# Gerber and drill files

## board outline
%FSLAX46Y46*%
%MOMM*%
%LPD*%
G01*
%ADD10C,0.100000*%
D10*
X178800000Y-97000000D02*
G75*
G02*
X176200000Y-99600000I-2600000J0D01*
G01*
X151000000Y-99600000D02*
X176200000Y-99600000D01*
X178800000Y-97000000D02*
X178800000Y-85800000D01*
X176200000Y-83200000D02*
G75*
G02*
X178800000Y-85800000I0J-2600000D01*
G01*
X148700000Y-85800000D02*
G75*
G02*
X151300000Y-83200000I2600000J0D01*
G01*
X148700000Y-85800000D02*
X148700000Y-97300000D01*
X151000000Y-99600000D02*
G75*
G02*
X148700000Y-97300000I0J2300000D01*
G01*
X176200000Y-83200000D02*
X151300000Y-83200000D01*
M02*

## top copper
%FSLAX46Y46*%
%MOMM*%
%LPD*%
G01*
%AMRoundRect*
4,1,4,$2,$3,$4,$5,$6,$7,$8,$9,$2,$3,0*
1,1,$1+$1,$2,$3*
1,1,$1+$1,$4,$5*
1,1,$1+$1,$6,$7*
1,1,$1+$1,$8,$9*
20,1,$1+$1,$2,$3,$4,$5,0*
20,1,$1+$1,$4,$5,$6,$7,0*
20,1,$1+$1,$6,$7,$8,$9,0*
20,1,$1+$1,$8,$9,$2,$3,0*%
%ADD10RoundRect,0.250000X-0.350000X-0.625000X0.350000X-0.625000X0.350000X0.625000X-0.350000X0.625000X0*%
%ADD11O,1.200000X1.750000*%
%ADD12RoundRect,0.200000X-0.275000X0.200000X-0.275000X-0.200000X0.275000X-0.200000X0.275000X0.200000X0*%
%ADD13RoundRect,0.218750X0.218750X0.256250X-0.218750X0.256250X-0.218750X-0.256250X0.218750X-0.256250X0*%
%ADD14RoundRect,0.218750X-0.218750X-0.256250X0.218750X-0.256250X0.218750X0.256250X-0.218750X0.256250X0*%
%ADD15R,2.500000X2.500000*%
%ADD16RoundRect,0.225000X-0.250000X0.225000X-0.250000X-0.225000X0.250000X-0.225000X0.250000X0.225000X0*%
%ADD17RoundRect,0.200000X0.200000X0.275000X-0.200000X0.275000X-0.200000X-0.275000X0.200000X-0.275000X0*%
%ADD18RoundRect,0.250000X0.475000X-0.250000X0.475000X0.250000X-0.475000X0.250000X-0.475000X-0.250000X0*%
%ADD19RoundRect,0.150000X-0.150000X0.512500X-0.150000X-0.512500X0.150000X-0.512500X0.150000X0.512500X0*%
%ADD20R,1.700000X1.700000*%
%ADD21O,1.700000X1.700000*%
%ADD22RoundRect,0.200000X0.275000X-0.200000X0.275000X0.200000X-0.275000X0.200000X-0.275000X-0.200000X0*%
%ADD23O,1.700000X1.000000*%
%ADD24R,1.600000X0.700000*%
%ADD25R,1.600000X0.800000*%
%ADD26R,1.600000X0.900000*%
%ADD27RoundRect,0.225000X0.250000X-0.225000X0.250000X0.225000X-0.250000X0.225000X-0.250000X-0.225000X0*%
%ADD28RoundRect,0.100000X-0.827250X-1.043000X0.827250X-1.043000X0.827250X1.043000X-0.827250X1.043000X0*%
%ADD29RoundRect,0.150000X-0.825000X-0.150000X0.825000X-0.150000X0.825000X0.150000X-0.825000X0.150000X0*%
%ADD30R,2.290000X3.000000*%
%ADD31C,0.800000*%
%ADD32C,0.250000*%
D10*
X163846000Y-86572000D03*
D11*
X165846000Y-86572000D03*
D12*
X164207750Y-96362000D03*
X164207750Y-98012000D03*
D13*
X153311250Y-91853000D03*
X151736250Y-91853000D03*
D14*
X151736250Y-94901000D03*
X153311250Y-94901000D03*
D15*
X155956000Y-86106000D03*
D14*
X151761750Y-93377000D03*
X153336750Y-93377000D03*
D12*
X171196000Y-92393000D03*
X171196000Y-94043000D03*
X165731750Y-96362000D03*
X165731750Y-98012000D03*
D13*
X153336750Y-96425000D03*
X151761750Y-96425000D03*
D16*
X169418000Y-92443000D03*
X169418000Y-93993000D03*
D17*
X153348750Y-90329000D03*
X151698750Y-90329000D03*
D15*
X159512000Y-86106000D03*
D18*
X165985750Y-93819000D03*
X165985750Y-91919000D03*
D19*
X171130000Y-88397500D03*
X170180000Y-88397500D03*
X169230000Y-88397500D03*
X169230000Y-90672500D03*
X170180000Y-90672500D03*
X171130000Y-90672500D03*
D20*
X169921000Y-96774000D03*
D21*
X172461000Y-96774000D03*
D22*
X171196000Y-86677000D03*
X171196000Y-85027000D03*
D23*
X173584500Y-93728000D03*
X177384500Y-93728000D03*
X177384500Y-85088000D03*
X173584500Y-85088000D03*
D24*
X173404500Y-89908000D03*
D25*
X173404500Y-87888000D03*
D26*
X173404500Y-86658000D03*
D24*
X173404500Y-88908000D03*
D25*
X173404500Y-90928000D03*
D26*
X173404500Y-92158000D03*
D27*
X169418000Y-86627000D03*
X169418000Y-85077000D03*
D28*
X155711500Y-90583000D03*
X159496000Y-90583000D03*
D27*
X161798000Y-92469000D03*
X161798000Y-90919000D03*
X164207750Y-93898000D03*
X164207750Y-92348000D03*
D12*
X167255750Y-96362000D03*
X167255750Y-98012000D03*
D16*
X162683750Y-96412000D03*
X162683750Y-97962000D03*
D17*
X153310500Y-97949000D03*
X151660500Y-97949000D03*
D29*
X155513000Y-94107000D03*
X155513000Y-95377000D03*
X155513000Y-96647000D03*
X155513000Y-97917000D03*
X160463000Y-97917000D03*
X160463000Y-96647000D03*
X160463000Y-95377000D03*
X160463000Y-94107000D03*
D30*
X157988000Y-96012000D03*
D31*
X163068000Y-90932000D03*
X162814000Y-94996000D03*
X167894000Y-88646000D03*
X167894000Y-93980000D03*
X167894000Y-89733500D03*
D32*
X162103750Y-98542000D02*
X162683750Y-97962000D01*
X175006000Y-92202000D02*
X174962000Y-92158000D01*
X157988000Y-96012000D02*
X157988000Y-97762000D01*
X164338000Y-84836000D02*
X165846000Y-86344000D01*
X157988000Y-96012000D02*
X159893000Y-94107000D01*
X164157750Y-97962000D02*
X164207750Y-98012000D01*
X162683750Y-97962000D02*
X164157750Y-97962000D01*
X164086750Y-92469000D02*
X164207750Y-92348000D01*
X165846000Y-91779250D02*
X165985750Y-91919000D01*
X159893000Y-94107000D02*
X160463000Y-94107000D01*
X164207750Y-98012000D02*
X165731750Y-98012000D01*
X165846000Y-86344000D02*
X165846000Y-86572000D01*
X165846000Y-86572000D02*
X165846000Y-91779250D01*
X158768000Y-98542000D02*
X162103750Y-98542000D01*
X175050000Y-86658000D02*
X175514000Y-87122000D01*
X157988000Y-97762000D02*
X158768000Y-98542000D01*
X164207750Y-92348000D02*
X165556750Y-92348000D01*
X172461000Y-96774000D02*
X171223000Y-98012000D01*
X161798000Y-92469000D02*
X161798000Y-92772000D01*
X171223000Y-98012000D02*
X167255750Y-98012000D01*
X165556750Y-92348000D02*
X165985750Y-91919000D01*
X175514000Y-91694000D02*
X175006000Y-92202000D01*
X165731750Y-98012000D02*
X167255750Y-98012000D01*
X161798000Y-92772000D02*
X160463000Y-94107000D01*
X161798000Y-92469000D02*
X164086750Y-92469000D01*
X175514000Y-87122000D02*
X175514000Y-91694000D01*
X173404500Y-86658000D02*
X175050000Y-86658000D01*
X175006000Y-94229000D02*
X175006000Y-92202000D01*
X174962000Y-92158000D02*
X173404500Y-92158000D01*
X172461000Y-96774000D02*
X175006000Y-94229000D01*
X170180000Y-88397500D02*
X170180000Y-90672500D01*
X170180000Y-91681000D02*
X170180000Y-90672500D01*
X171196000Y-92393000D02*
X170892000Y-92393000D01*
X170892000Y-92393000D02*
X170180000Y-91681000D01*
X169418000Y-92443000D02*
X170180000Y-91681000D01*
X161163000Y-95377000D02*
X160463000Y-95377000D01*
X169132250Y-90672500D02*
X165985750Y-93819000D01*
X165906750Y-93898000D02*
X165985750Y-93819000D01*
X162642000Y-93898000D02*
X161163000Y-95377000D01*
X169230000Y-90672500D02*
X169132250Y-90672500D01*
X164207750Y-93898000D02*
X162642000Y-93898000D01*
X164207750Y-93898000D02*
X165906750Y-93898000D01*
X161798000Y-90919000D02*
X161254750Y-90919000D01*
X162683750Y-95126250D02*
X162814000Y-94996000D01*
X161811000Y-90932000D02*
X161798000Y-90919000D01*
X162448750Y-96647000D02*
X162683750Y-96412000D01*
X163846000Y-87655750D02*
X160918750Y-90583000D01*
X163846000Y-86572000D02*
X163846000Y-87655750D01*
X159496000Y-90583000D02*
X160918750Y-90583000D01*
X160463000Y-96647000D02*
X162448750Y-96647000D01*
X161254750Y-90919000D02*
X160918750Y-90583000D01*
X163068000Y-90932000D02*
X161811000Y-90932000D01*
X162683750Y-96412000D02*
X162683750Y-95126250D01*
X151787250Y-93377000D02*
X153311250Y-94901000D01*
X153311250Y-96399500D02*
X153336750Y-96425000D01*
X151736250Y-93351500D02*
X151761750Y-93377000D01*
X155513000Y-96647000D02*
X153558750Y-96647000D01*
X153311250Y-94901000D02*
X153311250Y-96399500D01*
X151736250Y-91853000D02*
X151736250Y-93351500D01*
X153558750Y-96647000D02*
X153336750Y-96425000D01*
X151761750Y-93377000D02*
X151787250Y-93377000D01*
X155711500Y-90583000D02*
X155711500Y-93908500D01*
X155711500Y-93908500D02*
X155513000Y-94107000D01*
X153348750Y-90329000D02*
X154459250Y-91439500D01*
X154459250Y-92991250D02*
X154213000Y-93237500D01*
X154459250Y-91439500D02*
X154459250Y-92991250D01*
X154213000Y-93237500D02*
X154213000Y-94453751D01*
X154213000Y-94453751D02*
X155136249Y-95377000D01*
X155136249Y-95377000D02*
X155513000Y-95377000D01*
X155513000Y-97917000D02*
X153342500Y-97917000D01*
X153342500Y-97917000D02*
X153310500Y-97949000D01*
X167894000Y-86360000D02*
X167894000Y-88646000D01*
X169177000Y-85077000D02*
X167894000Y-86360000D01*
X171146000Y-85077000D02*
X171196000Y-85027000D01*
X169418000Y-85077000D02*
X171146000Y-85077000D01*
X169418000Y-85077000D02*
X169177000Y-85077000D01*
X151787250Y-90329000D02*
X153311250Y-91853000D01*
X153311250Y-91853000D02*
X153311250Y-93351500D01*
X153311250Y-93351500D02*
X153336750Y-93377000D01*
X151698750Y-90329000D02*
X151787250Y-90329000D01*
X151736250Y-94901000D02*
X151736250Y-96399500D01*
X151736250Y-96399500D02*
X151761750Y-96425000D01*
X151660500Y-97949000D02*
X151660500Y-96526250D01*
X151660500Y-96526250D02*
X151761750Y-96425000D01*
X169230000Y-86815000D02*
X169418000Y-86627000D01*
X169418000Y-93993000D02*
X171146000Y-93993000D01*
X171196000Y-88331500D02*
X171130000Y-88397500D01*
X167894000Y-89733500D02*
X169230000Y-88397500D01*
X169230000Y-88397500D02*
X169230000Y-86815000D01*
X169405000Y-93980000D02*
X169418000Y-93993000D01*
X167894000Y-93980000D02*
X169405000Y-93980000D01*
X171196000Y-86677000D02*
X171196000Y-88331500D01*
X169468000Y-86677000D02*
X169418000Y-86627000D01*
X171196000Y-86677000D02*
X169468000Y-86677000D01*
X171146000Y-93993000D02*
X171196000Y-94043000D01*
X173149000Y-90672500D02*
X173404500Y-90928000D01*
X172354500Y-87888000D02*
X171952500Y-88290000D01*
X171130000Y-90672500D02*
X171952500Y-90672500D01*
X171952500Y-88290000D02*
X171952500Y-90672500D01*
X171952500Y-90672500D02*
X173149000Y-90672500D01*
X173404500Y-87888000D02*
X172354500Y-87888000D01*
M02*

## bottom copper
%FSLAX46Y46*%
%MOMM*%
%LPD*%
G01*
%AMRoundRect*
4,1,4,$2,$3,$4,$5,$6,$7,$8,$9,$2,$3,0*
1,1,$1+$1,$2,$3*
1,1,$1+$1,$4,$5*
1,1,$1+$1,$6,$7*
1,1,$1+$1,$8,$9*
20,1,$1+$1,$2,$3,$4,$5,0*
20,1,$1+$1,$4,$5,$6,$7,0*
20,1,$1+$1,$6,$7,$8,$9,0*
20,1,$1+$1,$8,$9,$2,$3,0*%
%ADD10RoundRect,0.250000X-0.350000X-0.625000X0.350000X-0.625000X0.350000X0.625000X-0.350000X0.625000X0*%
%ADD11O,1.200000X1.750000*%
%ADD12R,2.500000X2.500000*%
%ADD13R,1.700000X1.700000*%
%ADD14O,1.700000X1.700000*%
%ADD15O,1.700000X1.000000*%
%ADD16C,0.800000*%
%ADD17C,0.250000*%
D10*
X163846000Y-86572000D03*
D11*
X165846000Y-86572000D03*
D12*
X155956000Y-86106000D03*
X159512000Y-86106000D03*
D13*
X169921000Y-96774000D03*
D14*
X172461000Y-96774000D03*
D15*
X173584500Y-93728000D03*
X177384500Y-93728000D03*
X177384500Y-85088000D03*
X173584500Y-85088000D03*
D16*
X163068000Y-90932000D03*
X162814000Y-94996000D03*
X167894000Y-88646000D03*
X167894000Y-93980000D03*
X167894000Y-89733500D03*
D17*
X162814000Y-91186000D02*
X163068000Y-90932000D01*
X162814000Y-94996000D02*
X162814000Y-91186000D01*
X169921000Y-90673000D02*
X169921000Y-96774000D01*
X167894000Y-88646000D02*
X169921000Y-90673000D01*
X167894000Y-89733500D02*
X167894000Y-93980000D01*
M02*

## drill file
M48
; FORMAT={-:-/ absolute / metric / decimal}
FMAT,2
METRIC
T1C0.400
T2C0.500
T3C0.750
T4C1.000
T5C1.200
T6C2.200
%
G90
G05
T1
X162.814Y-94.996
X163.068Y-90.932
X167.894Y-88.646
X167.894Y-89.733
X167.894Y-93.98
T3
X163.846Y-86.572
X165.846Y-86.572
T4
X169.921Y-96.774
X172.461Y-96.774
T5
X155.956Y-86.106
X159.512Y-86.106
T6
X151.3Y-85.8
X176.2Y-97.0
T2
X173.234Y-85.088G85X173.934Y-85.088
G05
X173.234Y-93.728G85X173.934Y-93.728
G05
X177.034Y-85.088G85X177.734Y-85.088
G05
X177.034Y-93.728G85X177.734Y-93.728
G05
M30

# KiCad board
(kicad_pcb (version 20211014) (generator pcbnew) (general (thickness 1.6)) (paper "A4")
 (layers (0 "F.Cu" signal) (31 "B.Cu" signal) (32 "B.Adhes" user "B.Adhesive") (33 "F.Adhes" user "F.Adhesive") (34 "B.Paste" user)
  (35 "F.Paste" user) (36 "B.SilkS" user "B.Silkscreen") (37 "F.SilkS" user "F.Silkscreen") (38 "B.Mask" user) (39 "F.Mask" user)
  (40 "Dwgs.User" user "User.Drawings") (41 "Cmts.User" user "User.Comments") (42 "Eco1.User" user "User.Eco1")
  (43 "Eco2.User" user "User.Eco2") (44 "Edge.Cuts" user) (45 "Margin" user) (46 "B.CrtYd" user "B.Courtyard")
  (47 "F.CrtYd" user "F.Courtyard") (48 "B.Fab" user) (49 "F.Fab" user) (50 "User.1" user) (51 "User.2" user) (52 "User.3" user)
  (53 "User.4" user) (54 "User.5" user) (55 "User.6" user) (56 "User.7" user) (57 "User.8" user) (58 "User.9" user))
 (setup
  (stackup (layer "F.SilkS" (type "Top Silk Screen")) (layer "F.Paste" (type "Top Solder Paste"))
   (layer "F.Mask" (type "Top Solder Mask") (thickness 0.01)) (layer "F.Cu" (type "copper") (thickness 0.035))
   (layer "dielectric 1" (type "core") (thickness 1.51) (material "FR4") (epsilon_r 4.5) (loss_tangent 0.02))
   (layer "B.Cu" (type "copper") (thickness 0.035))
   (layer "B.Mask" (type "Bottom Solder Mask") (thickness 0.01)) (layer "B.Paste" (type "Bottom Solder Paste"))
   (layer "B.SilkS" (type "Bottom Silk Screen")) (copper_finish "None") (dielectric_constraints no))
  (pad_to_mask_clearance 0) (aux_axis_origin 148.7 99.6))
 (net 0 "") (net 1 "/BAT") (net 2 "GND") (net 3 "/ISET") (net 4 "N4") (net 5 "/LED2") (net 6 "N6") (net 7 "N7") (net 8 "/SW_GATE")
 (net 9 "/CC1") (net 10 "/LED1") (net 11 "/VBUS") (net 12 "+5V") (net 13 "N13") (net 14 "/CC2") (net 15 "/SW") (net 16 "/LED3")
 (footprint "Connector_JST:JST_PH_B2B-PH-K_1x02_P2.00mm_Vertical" (layer "F.Cu") (at 163.846 86.572)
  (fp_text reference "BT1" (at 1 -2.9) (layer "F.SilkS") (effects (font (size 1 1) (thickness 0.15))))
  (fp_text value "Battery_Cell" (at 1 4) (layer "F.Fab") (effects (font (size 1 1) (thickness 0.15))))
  (pad "1" thru_hole roundrect (at 0 0) (size 1.2 1.75) (drill 0.75) (layers *.Cu *.Mask) (roundrect_rratio 0.208333) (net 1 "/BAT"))
  (pad "2" thru_hole oval (at 2 0) (size 1.2 1.75) (drill 0.75) (layers *.Cu *.Mask) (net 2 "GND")))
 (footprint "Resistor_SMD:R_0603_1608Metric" (layer "F.Cu") (at 164.20775 97.187 -90)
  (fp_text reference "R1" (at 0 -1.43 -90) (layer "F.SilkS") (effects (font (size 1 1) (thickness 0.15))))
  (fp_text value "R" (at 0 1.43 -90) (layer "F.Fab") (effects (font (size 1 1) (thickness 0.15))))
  (pad "1" smd roundrect (at -0.825 0 270) (size 0.8 0.95) (layers "F.Cu" "F.Paste" "F.Mask") (roundrect_rratio 0.25) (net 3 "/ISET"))
  (pad "2" smd roundrect (at 0.825 0 270) (size 0.8 0.95) (layers "F.Cu" "F.Paste" "F.Mask") (roundrect_rratio 0.25) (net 2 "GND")))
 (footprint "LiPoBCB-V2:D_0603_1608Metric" (layer "F.Cu") (at 152.52375 91.853 180)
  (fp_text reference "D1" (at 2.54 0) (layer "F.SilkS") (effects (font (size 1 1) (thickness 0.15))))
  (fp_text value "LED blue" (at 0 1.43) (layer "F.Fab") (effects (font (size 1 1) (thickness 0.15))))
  (pad "1" smd roundrect (at -0.7875 0 180) (size 0.875 0.95) (layers "F.Cu" "F.Paste" "F.Mask") (roundrect_rratio 0.25) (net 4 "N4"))
  (pad "2" smd roundrect (at 0.7875 0 180) (size 0.875 0.95) (layers "F.Cu" "F.Paste" "F.Mask") (roundrect_rratio 0.25) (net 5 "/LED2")))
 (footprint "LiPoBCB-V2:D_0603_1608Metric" (layer "F.Cu") (at 152.52375 94.901)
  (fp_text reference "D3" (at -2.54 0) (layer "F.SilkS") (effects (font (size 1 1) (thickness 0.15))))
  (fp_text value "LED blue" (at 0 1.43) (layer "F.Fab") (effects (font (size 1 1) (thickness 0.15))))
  (pad "1" smd roundrect (at -0.7875 0) (size 0.875 0.95) (layers "F.Cu" "F.Paste" "F.Mask") (roundrect_rratio 0.25) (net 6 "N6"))
  (pad "2" smd roundrect (at 0.7875 0) (size 0.875 0.95) (layers "F.Cu" "F.Paste" "F.Mask") (roundrect_rratio 0.25) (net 5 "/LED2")))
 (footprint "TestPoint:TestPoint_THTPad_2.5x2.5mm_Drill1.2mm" (layer "F.Cu") (at 155.956 86.106)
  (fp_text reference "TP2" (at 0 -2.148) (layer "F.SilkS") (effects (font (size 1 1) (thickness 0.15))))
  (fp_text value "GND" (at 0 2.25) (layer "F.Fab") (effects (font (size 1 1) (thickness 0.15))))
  (pad "1" thru_hole rect (at 0 0) (size 2.5 2.5) (drill 1.2) (layers *.Cu *.Mask) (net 2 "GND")))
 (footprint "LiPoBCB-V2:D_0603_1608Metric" (layer "F.Cu") (at 152.54925 93.377)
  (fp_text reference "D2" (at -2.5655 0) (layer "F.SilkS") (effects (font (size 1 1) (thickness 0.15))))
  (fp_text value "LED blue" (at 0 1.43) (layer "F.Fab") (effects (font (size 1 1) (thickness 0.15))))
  (pad "1" smd roundrect (at -0.7875 0) (size 0.875 0.95) (layers "F.Cu" "F.Paste" "F.Mask") (roundrect_rratio 0.25) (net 5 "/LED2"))
  (pad "2" smd roundrect (at 0.7875 0) (size 0.875 0.95) (layers "F.Cu" "F.Paste" "F.Mask") (roundrect_rratio 0.25) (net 4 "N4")))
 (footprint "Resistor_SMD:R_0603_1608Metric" (layer "F.Cu") (at 171.196 93.218 -90)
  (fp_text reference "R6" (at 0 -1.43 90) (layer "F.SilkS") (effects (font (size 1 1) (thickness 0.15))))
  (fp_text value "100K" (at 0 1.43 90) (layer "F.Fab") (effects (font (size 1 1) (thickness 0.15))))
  (pad "1" smd roundrect (at -0.825 0 270) (size 0.8 0.95) (layers "F.Cu" "F.Paste" "F.Mask") (roundrect_rratio 0.25) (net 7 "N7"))
  (pad "2" smd roundrect (at 0.825 0 270) (size 0.8 0.95) (layers "F.Cu" "F.Paste" "F.Mask") (roundrect_rratio 0.25) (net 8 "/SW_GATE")))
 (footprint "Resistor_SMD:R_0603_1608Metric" (layer "F.Cu") (at 165.73175 97.187 -90)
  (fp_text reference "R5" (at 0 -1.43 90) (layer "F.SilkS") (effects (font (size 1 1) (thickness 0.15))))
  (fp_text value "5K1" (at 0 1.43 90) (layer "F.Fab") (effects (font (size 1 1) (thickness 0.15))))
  (pad "1" smd roundrect (at -0.825 0 270) (size 0.8 0.95) (layers "F.Cu" "F.Paste" "F.Mask") (roundrect_rratio 0.25) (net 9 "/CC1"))
  (pad "2" smd roundrect (at 0.825 0 270) (size 0.8 0.95) (layers "F.Cu" "F.Paste" "F.Mask") (roundrect_rratio 0.25) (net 2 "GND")))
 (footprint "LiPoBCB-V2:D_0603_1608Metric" (layer "F.Cu") (at 152.54925 96.425 180)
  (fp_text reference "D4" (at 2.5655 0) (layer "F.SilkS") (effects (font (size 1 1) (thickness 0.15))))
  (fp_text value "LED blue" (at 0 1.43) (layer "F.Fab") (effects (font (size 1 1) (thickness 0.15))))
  (pad "1" smd roundrect (at -0.7875 0 180) (size 0.875 0.95) (layers "F.Cu" "F.Paste" "F.Mask") (roundrect_rratio 0.25) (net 5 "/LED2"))
  (pad "2" smd roundrect (at 0.7875 0 180) (size 0.875 0.95) (layers "F.Cu" "F.Paste" "F.Mask") (roundrect_rratio 0.25) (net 6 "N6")))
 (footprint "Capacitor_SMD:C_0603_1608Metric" (layer "F.Cu") (at 169.418 93.218 -90)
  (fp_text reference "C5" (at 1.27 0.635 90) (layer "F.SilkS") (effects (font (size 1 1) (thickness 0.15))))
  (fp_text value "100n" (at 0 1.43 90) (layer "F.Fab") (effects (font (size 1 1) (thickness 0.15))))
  (pad "1" smd roundrect (at -0.775 0 270) (size 0.9 0.95) (layers "F.Cu" "F.Paste" "F.Mask") (roundrect_rratio 0.25) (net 7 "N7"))
  (pad "2" smd roundrect (at 0.775 0 270) (size 0.9 0.95) (layers "F.Cu" "F.Paste" "F.Mask") (roundrect_rratio 0.25) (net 8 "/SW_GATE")))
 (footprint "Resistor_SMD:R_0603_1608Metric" (layer "F.Cu") (at 152.52375 90.329 180)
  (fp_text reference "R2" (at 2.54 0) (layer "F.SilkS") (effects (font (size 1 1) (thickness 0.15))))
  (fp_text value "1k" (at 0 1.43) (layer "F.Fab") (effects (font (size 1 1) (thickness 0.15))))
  (pad "1" smd roundrect (at -0.825 0 180) (size 0.8 0.95) (layers "F.Cu" "F.Paste" "F.Mask") (roundrect_rratio 0.25) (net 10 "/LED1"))
  (pad "2" smd roundrect (at 0.825 0 180) (size 0.8 0.95) (layers "F.Cu" "F.Paste" "F.Mask") (roundrect_rratio 0.25) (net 4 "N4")))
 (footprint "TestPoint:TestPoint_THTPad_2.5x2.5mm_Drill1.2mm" (layer "F.Cu") (at 159.512 86.106)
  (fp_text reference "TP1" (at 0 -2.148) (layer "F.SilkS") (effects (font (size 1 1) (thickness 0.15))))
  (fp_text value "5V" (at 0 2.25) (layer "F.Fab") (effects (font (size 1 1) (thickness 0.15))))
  (pad "1" thru_hole rect (at 0 0) (size 2.5 2.5) (drill 1.2) (layers *.Cu *.Mask) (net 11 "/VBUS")))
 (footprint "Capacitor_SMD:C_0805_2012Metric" (layer "F.Cu") (at 165.98575 92.869 90)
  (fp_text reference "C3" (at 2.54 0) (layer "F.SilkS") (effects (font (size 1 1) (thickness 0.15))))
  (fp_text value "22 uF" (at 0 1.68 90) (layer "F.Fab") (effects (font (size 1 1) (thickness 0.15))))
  (pad "1" smd roundrect (at -0.95 0 90) (size 1 1.45) (layers "F.Cu" "F.Paste" "F.Mask") (roundrect_rratio 0.25) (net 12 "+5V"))
  (pad "2" smd roundrect (at 0.95 0 90) (size 1 1.45) (layers "F.Cu" "F.Paste" "F.Mask") (roundrect_rratio 0.25) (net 2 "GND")))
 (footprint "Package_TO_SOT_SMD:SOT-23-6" (layer "F.Cu") (at 170.18 89.535 -90)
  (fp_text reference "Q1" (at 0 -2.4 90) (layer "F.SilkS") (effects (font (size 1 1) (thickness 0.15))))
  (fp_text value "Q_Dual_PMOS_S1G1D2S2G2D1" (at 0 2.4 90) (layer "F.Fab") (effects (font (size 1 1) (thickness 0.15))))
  (pad "1" smd roundrect (at -1.1375 -0.95 270) (size 1.325 0.6) (layers "F.Cu" "F.Paste" "F.Mask") (roundrect_rratio 0.25)
   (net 8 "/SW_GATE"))
  (pad "2" smd roundrect (at -1.1375 0 270) (size 1.325 0.6) (layers "F.Cu" "F.Paste" "F.Mask") (roundrect_rratio 0.25) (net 7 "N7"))
  (pad "3" smd roundrect (at -1.1375 0.95 270) (size 1.325 0.6) (layers "F.Cu" "F.Paste" "F.Mask") (roundrect_rratio 0.25)
   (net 8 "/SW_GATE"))
  (pad "4" smd roundrect (at 1.1375 0.95 270) (size 1.325 0.6) (layers "F.Cu" "F.Paste" "F.Mask") (roundrect_rratio 0.25) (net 12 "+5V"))
  (pad "5" smd roundrect (at 1.1375 0 270) (size 1.325 0.6) (layers "F.Cu" "F.Paste" "F.Mask") (roundrect_rratio 0.25) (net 7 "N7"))
  (pad "6" smd roundrect (at 1.1375 -0.95 270) (size 1.325 0.6) (layers "F.Cu" "F.Paste" "F.Mask") (roundrect_rratio 0.25) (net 11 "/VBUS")))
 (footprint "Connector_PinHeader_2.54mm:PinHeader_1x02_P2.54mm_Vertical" (layer "F.Cu") (at 169.921 96.774 90)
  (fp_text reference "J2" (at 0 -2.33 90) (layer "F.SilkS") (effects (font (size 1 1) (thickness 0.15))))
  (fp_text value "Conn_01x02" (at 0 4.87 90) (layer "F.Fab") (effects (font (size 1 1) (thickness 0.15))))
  (pad "1" thru_hole rect (at 0 0 90) (size 1.7 1.7) (drill 1) (layers *.Cu *.Mask) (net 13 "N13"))
  (pad "2" thru_hole oval (at 0 2.54 90) (size 1.7 1.7) (drill 1) (layers *.Cu *.Mask) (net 2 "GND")))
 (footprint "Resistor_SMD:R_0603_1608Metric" (layer "F.Cu") (at 171.196 85.852 90)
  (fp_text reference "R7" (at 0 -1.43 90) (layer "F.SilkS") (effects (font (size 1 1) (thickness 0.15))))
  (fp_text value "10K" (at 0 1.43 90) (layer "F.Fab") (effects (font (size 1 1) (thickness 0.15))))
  (pad "1" smd roundrect (at -0.825 0 90) (size 0.8 0.95) (layers "F.Cu" "F.Paste" "F.Mask") (roundrect_rratio 0.25) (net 8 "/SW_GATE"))
  (pad "2" smd roundrect (at 0.825 0 90) (size 0.8 0.95) (layers "F.Cu" "F.Paste" "F.Mask") (roundrect_rratio 0.25) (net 13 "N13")))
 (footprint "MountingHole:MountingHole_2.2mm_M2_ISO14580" (layer "F.Cu") (at 151.3 85.8)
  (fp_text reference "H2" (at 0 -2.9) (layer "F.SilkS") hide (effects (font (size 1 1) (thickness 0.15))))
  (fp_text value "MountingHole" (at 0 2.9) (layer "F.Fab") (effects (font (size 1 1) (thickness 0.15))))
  (pad "" np_thru_hole circle (at 0 0) (size 2.2 2.2) (drill 2.2) (layers *.Cu *.Mask)))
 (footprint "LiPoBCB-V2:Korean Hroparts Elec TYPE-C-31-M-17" (layer "F.Cu") (at 173.4045 89.408 90)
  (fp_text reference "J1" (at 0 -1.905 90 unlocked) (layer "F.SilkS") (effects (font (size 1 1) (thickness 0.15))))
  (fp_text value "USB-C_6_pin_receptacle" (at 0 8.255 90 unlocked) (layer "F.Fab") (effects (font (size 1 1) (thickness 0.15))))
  (pad "1" thru_hole oval (at -4.32 0.18 90) (size 1 1.7) (drill oval 0.5 1.2) (layers *.Cu *.Mask))
  (pad "2" thru_hole oval (at -4.32 3.98 90) (size 1 1.7) (drill oval 0.5 1.2) (layers *.Cu *.Mask))
  (pad "3" thru_hole oval (at 4.32 3.98 90) (size 1 1.7) (drill oval 0.5 1.2) (layers *.Cu *.Mask))
  (pad "4" thru_hole oval (at 4.32 0.18 90) (size 1 1.7) (drill oval 0.5 1.2) (layers *.Cu *.Mask))
  (pad "A5" smd rect (at -0.5 0 90) (size 0.7 1.6) (layers "F.Cu" "F.Paste" "F.Mask") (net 9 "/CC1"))
  (pad "A9" smd rect (at 1.52 0 90) (size 0.8 1.6) (layers "F.Cu" "F.Paste" "F.Mask") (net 11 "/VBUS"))
  (pad "A12" smd rect (at 2.75 0 90) (size 0.9 1.6) (layers "F.Cu" "F.Paste" "F.Mask") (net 2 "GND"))
  (pad "B5" smd rect (at 0.5 0 90) (size 0.7 1.6) (layers "F.Cu" "F.Paste" "F.Mask") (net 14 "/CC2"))
  (pad "B9" smd rect (at -1.52 0 90) (size 0.8 1.6) (layers "F.Cu" "F.Paste" "F.Mask") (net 11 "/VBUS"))
  (pad "B12" smd rect (at -2.75 0 90) (size 0.9 1.6) (layers "F.Cu" "F.Paste" "F.Mask") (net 2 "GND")))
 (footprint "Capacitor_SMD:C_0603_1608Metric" (layer "F.Cu") (at 169.418 85.852 90)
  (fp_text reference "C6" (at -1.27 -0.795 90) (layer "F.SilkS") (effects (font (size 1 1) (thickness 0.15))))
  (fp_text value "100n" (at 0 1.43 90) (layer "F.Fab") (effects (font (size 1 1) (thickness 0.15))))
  (pad "1" smd roundrect (at -0.775 0 90) (size 0.9 0.95) (layers "F.Cu" "F.Paste" "F.Mask") (roundrect_rratio 0.25) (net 8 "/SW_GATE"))
  (pad "2" smd roundrect (at 0.775 0 90) (size 0.9 0.95) (layers "F.Cu" "F.Paste" "F.Mask") (roundrect_rratio 0.25) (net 13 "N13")))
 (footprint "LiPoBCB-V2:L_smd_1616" (layer "F.Cu") (at 157.60375 90.583)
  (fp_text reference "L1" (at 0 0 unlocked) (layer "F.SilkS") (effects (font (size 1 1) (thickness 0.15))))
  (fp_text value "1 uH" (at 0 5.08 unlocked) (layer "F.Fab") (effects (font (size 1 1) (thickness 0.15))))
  (pad "1" smd roundrect (at -1.89225 0) (size 1.8545 2.286) (layers "F.Cu" "F.Paste" "F.Mask") (roundrect_rratio 0.05392289027)
   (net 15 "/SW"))
  (pad "2" smd roundrect (at 1.89225 0) (size 1.8545 2.286) (layers "F.Cu" "F.Paste" "F.Mask") (roundrect_rratio 0.05392289027)
   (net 1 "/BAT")))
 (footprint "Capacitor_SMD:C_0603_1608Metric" (layer "F.Cu") (at 161.798 91.694 90)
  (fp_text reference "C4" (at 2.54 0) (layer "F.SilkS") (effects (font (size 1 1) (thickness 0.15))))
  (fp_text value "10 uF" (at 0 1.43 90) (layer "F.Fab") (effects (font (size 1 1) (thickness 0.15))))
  (pad "1" smd roundrect (at -0.775 0 90) (size 0.9 0.95) (layers "F.Cu" "F.Paste" "F.Mask") (roundrect_rratio 0.25) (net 2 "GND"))
  (pad "2" smd roundrect (at 0.775 0 90) (size 0.9 0.95) (layers "F.Cu" "F.Paste" "F.Mask") (roundrect_rratio 0.25) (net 1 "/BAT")))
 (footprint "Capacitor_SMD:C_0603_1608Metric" (layer "F.Cu") (at 164.20775 93.123 90)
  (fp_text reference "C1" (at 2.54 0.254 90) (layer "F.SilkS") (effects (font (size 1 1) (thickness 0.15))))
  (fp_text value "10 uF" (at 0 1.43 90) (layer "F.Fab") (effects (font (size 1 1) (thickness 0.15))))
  (pad "1" smd roundrect (at -0.775 0 90) (size 0.9 0.95) (layers "F.Cu" "F.Paste" "F.Mask") (roundrect_rratio 0.25) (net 12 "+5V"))
  (pad "2" smd roundrect (at 0.775 0 90) (size 0.9 0.95) (layers "F.Cu" "F.Paste" "F.Mask") (roundrect_rratio 0.25) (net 2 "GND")))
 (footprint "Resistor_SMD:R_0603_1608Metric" (layer "F.Cu") (at 167.25575 97.187 -90)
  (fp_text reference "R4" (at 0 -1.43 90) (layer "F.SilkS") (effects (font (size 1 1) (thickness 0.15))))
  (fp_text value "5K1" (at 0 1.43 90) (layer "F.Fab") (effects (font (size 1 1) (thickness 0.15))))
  (pad "1" smd roundrect (at -0.825 0 270) (size 0.8 0.95) (layers "F.Cu" "F.Paste" "F.Mask") (roundrect_rratio 0.25) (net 14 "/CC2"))
  (pad "2" smd roundrect (at 0.825 0 270) (size 0.8 0.95) (layers "F.Cu" "F.Paste" "F.Mask") (roundrect_rratio 0.25) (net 2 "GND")))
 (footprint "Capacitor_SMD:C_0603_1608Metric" (layer "F.Cu") (at 162.68375 97.187 -90)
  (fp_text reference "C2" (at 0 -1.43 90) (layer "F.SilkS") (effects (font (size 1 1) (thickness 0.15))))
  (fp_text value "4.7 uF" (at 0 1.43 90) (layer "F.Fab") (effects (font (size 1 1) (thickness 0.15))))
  (pad "1" smd roundrect (at -0.775 0 270) (size 0.9 0.95) (layers "F.Cu" "F.Paste" "F.Mask") (roundrect_rratio 0.25) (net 1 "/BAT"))
  (pad "2" smd roundrect (at 0.775 0 270) (size 0.9 0.95) (layers "F.Cu" "F.Paste" "F.Mask") (roundrect_rratio 0.25) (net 2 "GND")))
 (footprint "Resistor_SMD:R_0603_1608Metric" (layer "F.Cu") (at 152.4855 97.949 180)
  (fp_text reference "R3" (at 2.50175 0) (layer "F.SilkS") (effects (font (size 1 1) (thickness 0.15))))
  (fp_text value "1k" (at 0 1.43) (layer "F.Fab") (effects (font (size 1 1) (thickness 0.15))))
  (pad "1" smd roundrect (at -0.825 0 180) (size 0.8 0.95) (layers "F.Cu" "F.Paste" "F.Mask") (roundrect_rratio 0.25) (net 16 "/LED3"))
  (pad "2" smd roundrect (at 0.825 0 180) (size 0.8 0.95) (layers "F.Cu" "F.Paste" "F.Mask") (roundrect_rratio 0.25) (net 6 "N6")))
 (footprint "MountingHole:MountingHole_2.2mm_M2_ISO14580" (layer "F.Cu") (at 176.2 97)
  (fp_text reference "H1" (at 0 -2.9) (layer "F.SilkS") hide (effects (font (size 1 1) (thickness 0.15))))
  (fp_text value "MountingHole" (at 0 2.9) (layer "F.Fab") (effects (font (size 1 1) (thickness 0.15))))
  (pad "" np_thru_hole circle (at 0 0) (size 2.2 2.2) (drill 2.2) (layers *.Cu *.Mask)))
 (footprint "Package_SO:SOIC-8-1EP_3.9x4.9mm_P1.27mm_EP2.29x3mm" (layer "F.Cu") (at 157.988 96.012)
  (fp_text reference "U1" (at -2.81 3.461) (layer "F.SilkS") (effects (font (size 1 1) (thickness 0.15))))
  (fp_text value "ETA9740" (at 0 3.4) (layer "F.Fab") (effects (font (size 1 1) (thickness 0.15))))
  (pad "" smd roundrect (at 0.57 -0.75) (size 0.92 1.21) (layers "F.Paste") (roundrect_rratio 0.25))
  (pad "" smd roundrect (at 0.57 0.75) (size 0.92 1.21) (layers "F.Paste") (roundrect_rratio 0.25))
  (pad "" smd roundrect (at -0.57 -0.75) (size 0.92 1.21) (layers "F.Paste") (roundrect_rratio 0.25))
  (pad "" smd roundrect (at -0.57 0.75) (size 0.92 1.21) (layers "F.Paste") (roundrect_rratio 0.25))
  (pad "1" smd roundrect (at -2.475 -1.905) (size 1.95 0.6) (layers "F.Cu" "F.Paste" "F.Mask") (roundrect_rratio 0.25) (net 15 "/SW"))
  (pad "2" smd roundrect (at -2.475 -0.635) (size 1.95 0.6) (layers "F.Cu" "F.Paste" "F.Mask") (roundrect_rratio 0.25) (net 10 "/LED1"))
  (pad "3" smd roundrect (at -2.475 0.635) (size 1.95 0.6) (layers "F.Cu" "F.Paste" "F.Mask") (roundrect_rratio 0.25) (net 5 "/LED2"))
  (pad "4" smd roundrect (at -2.475 1.905) (size 1.95 0.6) (layers "F.Cu" "F.Paste" "F.Mask") (roundrect_rratio 0.25) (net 16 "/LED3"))
  (pad "5" smd roundrect (at 2.475 1.905) (size 1.95 0.6) (layers "F.Cu" "F.Paste" "F.Mask") (roundrect_rratio 0.25) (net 3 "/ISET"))
  (pad "6" smd roundrect (at 2.475 0.635) (size 1.95 0.6) (layers "F.Cu" "F.Paste" "F.Mask") (roundrect_rratio 0.25) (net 1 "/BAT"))
  (pad "7" smd roundrect (at 2.475 -0.635) (size 1.95 0.6) (layers "F.Cu" "F.Paste" "F.Mask") (roundrect_rratio 0.25) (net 12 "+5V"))
  (pad "8" smd roundrect (at 2.475 -1.905) (size 1.95 0.6) (layers "F.Cu" "F.Paste" "F.Mask") (roundrect_rratio 0.25) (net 2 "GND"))
  (pad "9" smd rect (at 0 0) (size 2.29 3) (layers "F.Cu" "F.Mask") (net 2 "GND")))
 (gr_arc (start 178.8 97) (mid 178.038478 98.838478) (end 176.2 99.6) (layer "Edge.Cuts") (width 0.1))
 (gr_line (start 151 99.6) (end 176.2 99.6) (layer "Edge.Cuts") (width 0.1))
 (gr_line (start 178.8 97) (end 178.8 85.8) (layer "Edge.Cuts") (width 0.1))
 (gr_arc (start 176.2 83.2) (mid 178.038478 83.961522) (end 178.8 85.8) (layer "Edge.Cuts") (width 0.1))
 (gr_arc (start 148.7 85.8) (mid 149.461522 83.961522) (end 151.3 83.2) (layer "Edge.Cuts") (width 0.1))
 (gr_line (start 148.7 85.8) (end 148.7 97.3) (layer "Edge.Cuts") (width 0.1))
 (gr_arc (start 151 99.6) (mid 149.373654 98.926346) (end 148.7 97.3) (layer "Edge.Cuts") (width 0.1))
 (gr_line (start 176.2 83.2) (end 151.3 83.2) (layer "Edge.Cuts") (width 0.1))
 (segment (start 162.10375 98.542) (end 162.68375 97.962) (width 0.25) (layer "F.Cu") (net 2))
 (segment (start 175.006 92.202) (end 174.962 92.158) (width 0.25) (layer "F.Cu") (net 2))
 (segment (start 157.988 96.012) (end 157.988 97.762) (width 0.25) (layer "F.Cu") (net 2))
 (segment (start 164.338 84.836) (end 165.846 86.344) (width 0.25) (layer "F.Cu") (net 2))
 (segment (start 157.988 96.012) (end 159.893 94.107) (width 0.25) (layer "F.Cu") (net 2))
 (segment (start 164.15775 97.962) (end 164.20775 98.012) (width 0.25) (layer "F.Cu") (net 2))
 (segment (start 162.68375 97.962) (end 164.15775 97.962) (width 0.25) (layer "F.Cu") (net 2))
 (segment (start 164.08675 92.469) (end 164.20775 92.348) (width 0.25) (layer "F.Cu") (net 2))
 (segment (start 165.846 91.77925) (end 165.98575 91.919) (width 0.25) (layer "F.Cu") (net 2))
 (segment (start 159.893 94.107) (end 160.463 94.107) (width 0.25) (layer "F.Cu") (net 2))
 (segment (start 164.20775 98.012) (end 165.73175 98.012) (width 0.25) (layer "F.Cu") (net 2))
 (segment (start 165.846 86.344) (end 165.846 86.572) (width 0.25) (layer "F.Cu") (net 2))
 (segment (start 165.846 86.572) (end 165.846 91.77925) (width 0.25) (layer "F.Cu") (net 2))
 (segment (start 158.768 98.542) (end 162.10375 98.542) (width 0.25) (layer "F.Cu") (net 2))
 (segment (start 175.05 86.658) (end 175.514 87.122) (width 0.25) (layer "F.Cu") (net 2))
 (segment (start 157.988 97.762) (end 158.768 98.542) (width 0.25) (layer "F.Cu") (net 2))
 (segment (start 164.20775 92.348) (end 165.55675 92.348) (width 0.25) (layer "F.Cu") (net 2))
 (segment (start 172.461 96.774) (end 171.223 98.012) (width 0.25) (layer "F.Cu") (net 2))
 (segment (start 161.798 92.469) (end 161.798 92.772) (width 0.25) (layer "F.Cu") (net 2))
 (segment (start 171.223 98.012) (end 167.25575 98.012) (width 0.25) (layer "F.Cu") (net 2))
 (segment (start 165.55675 92.348) (end 165.98575 91.919) (width 0.25) (layer "F.Cu") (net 2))
 (segment (start 175.514 91.694) (end 175.006 92.202) (width 0.25) (layer "F.Cu") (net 2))
 (segment (start 165.73175 98.012) (end 167.25575 98.012) (width 0.25) (layer "F.Cu") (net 2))
 (segment (start 161.798 92.772) (end 160.463 94.107) (width 0.25) (layer "F.Cu") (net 2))
 (segment (start 161.798 92.469) (end 164.08675 92.469) (width 0.25) (layer "F.Cu") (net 2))
 (segment (start 175.514 87.122) (end 175.514 91.694) (width 0.25) (layer "F.Cu") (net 2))
 (segment (start 173.4045 86.658) (end 175.05 86.658) (width 0.25) (layer "F.Cu") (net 2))
 (segment (start 175.006 94.229) (end 175.006 92.202) (width 0.25) (layer "F.Cu") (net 2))
 (segment (start 174.962 92.158) (end 173.4045 92.158) (width 0.25) (layer "F.Cu") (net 2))
 (segment (start 172.461 96.774) (end 175.006 94.229) (width 0.25) (layer "F.Cu") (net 2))
 (segment (start 170.18 88.3975) (end 170.18 90.6725) (width 0.25) (layer "F.Cu") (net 7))
 (segment (start 170.18 91.681) (end 170.18 90.6725) (width 0.25) (layer "F.Cu") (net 7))
 (segment (start 171.196 92.393) (end 170.892 92.393) (width 0.25) (layer "F.Cu") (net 7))
 (segment (start 170.892 92.393) (end 170.18 91.681) (width 0.25) (layer "F.Cu") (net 7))
 (segment (start 169.418 92.443) (end 170.18 91.681) (width 0.25) (layer "F.Cu") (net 7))
 (segment (start 161.163 95.377) (end 160.463 95.377) (width 0.25) (layer "F.Cu") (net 12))
 (segment (start 169.13225 90.6725) (end 165.98575 93.819) (width 0.25) (layer "F.Cu") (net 12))
 (segment (start 165.90675 93.898) (end 165.98575 93.819) (width 0.25) (layer "F.Cu") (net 12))
 (segment (start 162.642 93.898) (end 161.163 95.377) (width 0.25) (layer "F.Cu") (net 12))
 (segment (start 169.23 90.6725) (end 169.13225 90.6725) (width 0.25) (layer "F.Cu") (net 12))
 (segment (start 164.20775 93.898) (end 162.642 93.898) (width 0.25) (layer "F.Cu") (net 12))
 (segment (start 164.20775 93.898) (end 165.90675 93.898) (width 0.25) (layer "F.Cu") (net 12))
 (segment (start 161.798 90.919) (end 161.25475 90.919) (width 0.25) (layer "F.Cu") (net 1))
 (segment (start 162.68375 95.12625) (end 162.814 94.996) (width 0.25) (layer "F.Cu") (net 1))
 (segment (start 161.811 90.932) (end 161.798 90.919) (width 0.25) (layer "F.Cu") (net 1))
 (segment (start 162.44875 96.647) (end 162.68375 96.412) (width 0.25) (layer "F.Cu") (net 1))
 (segment (start 163.846 87.65575) (end 160.91875 90.583) (width 0.25) (layer "F.Cu") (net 1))
 (segment (start 163.846 86.572) (end 163.846 87.65575) (width 0.25) (layer "F.Cu") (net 1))
 (segment (start 159.496 90.583) (end 160.91875 90.583) (width 0.25) (layer "F.Cu") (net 1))
 (segment (start 160.463 96.647) (end 162.44875 96.647) (width 0.25) (layer "F.Cu") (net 1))
 (segment (start 161.25475 90.919) (end 160.91875 90.583) (width 0.25) (layer "F.Cu") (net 1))
 (segment (start 163.068 90.932) (end 161.811 90.932) (width 0.25) (layer "F.Cu") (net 1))
 (segment (start 162.68375 96.412) (end 162.68375 95.12625) (width 0.25) (layer "F.Cu") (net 1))
 (via (at 163.068 90.932) (size 0.8) (drill 0.4) (layers "F.Cu" "B.Cu") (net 1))
 (via (at 162.814 94.996) (size 0.8) (drill 0.4) (layers "F.Cu" "B.Cu") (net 1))
 (segment (start 162.814 91.186) (end 163.068 90.932) (width 0.25) (layer "B.Cu") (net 1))
 (segment (start 162.814 94.996) (end 162.814 91.186) (width 0.25) (layer "B.Cu") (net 1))
 (segment (start 151.78725 93.377) (end 153.31125 94.901) (width 0.25) (layer "F.Cu") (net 5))
 (segment (start 153.31125 96.3995) (end 153.33675 96.425) (width 0.25) (layer "F.Cu") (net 5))
 (segment (start 151.73625 93.3515) (end 151.76175 93.377) (width 0.25) (layer "F.Cu") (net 5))
 (segment (start 155.513 96.647) (end 153.55875 96.647) (width 0.25) (layer "F.Cu") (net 5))
 (segment (start 153.31125 94.901) (end 153.31125 96.3995) (width 0.25) (layer "F.Cu") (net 5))
 (segment (start 151.73625 91.853) (end 151.73625 93.3515) (width 0.25) (layer "F.Cu") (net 5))
 (segment (start 153.55875 96.647) (end 153.33675 96.425) (width 0.25) (layer "F.Cu") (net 5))
 (segment (start 151.76175 93.377) (end 151.78725 93.377) (width 0.25) (layer "F.Cu") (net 5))
 (segment (start 155.7115 90.583) (end 155.7115 93.9085) (width 0.25) (layer "F.Cu") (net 15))
 (segment (start 155.7115 93.9085) (end 155.513 94.107) (width 0.25) (layer "F.Cu") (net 15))
 (segment (start 153.34875 90.329) (end 154.45925 91.4395) (width 0.25) (layer "F.Cu") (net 10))
 (segment (start 154.45925 92.99125) (end 154.213 93.2375) (width 0.25) (layer "F.Cu") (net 10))
 (segment (start 154.45925 91.4395) (end 154.45925 92.99125) (width 0.25) (layer "F.Cu") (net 10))
 (segment (start 154.213 93.2375) (end 154.213 94.453751) (width 0.25) (layer "F.Cu") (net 10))
 (segment (start 154.213 94.453751) (end 155.136249 95.377) (width 0.25) (layer "F.Cu") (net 10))
 (segment (start 155.136249 95.377) (end 155.513 95.377) (width 0.25) (layer "F.Cu") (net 10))
 (segment (start 155.513 97.917) (end 153.3425 97.917) (width 0.25) (layer "F.Cu") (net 16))
 (segment (start 153.3425 97.917) (end 153.3105 97.949) (width 0.25) (layer "F.Cu") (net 16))
 (segment (start 167.894 86.36) (end 167.894 88.646) (width 0.25) (layer "F.Cu") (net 13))
 (segment (start 169.177 85.077) (end 167.894 86.36) (width 0.25) (layer "F.Cu") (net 13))
 (segment (start 171.146 85.077) (end 171.196 85.027) (width 0.25) (layer "F.Cu") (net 13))
 (segment (start 169.418 85.077) (end 171.146 85.077) (width 0.25) (layer "F.Cu") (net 13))
 (segment (start 169.418 85.077) (end 169.177 85.077) (width 0.25) (layer "F.Cu") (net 13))
 (via (at 167.894 88.646) (size 0.8) (drill 0.4) (layers "F.Cu" "B.Cu") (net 13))
 (segment (start 169.921 90.673) (end 169.921 96.774) (width 0.25) (layer "B.Cu") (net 13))
 (segment (start 167.894 88.646) (end 169.921 90.673) (width 0.25) (layer "B.Cu") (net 13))
 (segment (start 151.78725 90.329) (end 153.31125 91.853) (width 0.25) (layer "F.Cu") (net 4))
 (segment (start 153.31125 91.853) (end 153.31125 93.3515) (width 0.25) (layer "F.Cu") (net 4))
 (segment (start 153.31125 93.3515) (end 153.33675 93.377) (width 0.25) (layer "F.Cu") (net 4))
 (segment (start 151.69875 90.329) (end 151.78725 90.329) (width 0.25) (layer "F.Cu") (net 4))
 (segment (start 151.73625 94.901) (end 151.73625 96.3995) (width 0.25) (layer "F.Cu") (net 6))
 (segment (start 151.73625 96.3995) (end 151.76175 96.425) (width 0.25) (layer "F.Cu") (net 6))
 (segment (start 151.6605 97.949) (end 151.6605 96.52625) (width 0.25) (layer "F.Cu") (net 6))
 (segment (start 151.6605 96.52625) (end 151.76175 96.425) (width 0.25) (layer "F.Cu") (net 6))
 (segment (start 169.23 86.815) (end 169.418 86.627) (width 0.25) (layer "F.Cu") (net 8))
 (segment (start 169.418 93.993) (end 171.146 93.993) (width 0.25) (layer "F.Cu") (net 8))
 (segment (start 171.196 88.3315) (end 171.13 88.3975) (width 0.25) (layer "F.Cu") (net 8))
 (segment (start 167.894 89.7335) (end 169.23 88.3975) (width 0.25) (layer "F.Cu") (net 8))
 (segment (start 169.23 88.3975) (end 169.23 86.815) (width 0.25) (layer "F.Cu") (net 8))
 (segment (start 169.405 93.98) (end 169.418 93.993) (width 0.25) (layer "F.Cu") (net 8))
 (segment (start 167.894 93.98) (end 169.405 93.98) (width 0.25) (layer "F.Cu") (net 8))
 (segment (start 171.196 86.677) (end 171.196 88.3315) (width 0.25) (layer "F.Cu") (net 8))
 (segment (start 169.468 86.677) (end 169.418 86.627) (width 0.25) (layer "F.Cu") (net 8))
 (segment (start 171.196 86.677) (end 169.468 86.677) (width 0.25) (layer "F.Cu") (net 8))
 (segment (start 171.146 93.993) (end 171.196 94.043) (width 0.25) (layer "F.Cu") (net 8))
 (via (at 167.894 93.98) (size 0.8) (drill 0.4) (layers "F.Cu" "B.Cu") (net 8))
 (via (at 167.894 89.7335) (size 0.8) (drill 0.4) (layers "F.Cu" "B.Cu") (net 8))
 (segment (start 167.894 89.7335) (end 167.894 93.98) (width 0.25) (layer "B.Cu") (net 8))
 (segment (start 173.149 90.6725) (end 173.4045 90.928) (width 0.25) (layer "F.Cu") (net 11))
 (segment (start 172.3545 87.888) (end 171.9525 88.29) (width 0.25) (layer "F.Cu") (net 11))
 (segment (start 171.13 90.6725) (end 171.9525 90.6725) (width 0.25) (layer "F.Cu") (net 11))
 (segment (start 171.9525 88.29) (end 171.9525 90.6725) (width 0.25) (layer "F.Cu") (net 11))
 (segment (start 171.9525 90.6725) (end 173.149 90.6725) (width 0.25) (layer "F.Cu") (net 11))
 (segment (start 173.4045 87.888) (end 172.3545 87.888) (width 0.25) (layer "F.Cu") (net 11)))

